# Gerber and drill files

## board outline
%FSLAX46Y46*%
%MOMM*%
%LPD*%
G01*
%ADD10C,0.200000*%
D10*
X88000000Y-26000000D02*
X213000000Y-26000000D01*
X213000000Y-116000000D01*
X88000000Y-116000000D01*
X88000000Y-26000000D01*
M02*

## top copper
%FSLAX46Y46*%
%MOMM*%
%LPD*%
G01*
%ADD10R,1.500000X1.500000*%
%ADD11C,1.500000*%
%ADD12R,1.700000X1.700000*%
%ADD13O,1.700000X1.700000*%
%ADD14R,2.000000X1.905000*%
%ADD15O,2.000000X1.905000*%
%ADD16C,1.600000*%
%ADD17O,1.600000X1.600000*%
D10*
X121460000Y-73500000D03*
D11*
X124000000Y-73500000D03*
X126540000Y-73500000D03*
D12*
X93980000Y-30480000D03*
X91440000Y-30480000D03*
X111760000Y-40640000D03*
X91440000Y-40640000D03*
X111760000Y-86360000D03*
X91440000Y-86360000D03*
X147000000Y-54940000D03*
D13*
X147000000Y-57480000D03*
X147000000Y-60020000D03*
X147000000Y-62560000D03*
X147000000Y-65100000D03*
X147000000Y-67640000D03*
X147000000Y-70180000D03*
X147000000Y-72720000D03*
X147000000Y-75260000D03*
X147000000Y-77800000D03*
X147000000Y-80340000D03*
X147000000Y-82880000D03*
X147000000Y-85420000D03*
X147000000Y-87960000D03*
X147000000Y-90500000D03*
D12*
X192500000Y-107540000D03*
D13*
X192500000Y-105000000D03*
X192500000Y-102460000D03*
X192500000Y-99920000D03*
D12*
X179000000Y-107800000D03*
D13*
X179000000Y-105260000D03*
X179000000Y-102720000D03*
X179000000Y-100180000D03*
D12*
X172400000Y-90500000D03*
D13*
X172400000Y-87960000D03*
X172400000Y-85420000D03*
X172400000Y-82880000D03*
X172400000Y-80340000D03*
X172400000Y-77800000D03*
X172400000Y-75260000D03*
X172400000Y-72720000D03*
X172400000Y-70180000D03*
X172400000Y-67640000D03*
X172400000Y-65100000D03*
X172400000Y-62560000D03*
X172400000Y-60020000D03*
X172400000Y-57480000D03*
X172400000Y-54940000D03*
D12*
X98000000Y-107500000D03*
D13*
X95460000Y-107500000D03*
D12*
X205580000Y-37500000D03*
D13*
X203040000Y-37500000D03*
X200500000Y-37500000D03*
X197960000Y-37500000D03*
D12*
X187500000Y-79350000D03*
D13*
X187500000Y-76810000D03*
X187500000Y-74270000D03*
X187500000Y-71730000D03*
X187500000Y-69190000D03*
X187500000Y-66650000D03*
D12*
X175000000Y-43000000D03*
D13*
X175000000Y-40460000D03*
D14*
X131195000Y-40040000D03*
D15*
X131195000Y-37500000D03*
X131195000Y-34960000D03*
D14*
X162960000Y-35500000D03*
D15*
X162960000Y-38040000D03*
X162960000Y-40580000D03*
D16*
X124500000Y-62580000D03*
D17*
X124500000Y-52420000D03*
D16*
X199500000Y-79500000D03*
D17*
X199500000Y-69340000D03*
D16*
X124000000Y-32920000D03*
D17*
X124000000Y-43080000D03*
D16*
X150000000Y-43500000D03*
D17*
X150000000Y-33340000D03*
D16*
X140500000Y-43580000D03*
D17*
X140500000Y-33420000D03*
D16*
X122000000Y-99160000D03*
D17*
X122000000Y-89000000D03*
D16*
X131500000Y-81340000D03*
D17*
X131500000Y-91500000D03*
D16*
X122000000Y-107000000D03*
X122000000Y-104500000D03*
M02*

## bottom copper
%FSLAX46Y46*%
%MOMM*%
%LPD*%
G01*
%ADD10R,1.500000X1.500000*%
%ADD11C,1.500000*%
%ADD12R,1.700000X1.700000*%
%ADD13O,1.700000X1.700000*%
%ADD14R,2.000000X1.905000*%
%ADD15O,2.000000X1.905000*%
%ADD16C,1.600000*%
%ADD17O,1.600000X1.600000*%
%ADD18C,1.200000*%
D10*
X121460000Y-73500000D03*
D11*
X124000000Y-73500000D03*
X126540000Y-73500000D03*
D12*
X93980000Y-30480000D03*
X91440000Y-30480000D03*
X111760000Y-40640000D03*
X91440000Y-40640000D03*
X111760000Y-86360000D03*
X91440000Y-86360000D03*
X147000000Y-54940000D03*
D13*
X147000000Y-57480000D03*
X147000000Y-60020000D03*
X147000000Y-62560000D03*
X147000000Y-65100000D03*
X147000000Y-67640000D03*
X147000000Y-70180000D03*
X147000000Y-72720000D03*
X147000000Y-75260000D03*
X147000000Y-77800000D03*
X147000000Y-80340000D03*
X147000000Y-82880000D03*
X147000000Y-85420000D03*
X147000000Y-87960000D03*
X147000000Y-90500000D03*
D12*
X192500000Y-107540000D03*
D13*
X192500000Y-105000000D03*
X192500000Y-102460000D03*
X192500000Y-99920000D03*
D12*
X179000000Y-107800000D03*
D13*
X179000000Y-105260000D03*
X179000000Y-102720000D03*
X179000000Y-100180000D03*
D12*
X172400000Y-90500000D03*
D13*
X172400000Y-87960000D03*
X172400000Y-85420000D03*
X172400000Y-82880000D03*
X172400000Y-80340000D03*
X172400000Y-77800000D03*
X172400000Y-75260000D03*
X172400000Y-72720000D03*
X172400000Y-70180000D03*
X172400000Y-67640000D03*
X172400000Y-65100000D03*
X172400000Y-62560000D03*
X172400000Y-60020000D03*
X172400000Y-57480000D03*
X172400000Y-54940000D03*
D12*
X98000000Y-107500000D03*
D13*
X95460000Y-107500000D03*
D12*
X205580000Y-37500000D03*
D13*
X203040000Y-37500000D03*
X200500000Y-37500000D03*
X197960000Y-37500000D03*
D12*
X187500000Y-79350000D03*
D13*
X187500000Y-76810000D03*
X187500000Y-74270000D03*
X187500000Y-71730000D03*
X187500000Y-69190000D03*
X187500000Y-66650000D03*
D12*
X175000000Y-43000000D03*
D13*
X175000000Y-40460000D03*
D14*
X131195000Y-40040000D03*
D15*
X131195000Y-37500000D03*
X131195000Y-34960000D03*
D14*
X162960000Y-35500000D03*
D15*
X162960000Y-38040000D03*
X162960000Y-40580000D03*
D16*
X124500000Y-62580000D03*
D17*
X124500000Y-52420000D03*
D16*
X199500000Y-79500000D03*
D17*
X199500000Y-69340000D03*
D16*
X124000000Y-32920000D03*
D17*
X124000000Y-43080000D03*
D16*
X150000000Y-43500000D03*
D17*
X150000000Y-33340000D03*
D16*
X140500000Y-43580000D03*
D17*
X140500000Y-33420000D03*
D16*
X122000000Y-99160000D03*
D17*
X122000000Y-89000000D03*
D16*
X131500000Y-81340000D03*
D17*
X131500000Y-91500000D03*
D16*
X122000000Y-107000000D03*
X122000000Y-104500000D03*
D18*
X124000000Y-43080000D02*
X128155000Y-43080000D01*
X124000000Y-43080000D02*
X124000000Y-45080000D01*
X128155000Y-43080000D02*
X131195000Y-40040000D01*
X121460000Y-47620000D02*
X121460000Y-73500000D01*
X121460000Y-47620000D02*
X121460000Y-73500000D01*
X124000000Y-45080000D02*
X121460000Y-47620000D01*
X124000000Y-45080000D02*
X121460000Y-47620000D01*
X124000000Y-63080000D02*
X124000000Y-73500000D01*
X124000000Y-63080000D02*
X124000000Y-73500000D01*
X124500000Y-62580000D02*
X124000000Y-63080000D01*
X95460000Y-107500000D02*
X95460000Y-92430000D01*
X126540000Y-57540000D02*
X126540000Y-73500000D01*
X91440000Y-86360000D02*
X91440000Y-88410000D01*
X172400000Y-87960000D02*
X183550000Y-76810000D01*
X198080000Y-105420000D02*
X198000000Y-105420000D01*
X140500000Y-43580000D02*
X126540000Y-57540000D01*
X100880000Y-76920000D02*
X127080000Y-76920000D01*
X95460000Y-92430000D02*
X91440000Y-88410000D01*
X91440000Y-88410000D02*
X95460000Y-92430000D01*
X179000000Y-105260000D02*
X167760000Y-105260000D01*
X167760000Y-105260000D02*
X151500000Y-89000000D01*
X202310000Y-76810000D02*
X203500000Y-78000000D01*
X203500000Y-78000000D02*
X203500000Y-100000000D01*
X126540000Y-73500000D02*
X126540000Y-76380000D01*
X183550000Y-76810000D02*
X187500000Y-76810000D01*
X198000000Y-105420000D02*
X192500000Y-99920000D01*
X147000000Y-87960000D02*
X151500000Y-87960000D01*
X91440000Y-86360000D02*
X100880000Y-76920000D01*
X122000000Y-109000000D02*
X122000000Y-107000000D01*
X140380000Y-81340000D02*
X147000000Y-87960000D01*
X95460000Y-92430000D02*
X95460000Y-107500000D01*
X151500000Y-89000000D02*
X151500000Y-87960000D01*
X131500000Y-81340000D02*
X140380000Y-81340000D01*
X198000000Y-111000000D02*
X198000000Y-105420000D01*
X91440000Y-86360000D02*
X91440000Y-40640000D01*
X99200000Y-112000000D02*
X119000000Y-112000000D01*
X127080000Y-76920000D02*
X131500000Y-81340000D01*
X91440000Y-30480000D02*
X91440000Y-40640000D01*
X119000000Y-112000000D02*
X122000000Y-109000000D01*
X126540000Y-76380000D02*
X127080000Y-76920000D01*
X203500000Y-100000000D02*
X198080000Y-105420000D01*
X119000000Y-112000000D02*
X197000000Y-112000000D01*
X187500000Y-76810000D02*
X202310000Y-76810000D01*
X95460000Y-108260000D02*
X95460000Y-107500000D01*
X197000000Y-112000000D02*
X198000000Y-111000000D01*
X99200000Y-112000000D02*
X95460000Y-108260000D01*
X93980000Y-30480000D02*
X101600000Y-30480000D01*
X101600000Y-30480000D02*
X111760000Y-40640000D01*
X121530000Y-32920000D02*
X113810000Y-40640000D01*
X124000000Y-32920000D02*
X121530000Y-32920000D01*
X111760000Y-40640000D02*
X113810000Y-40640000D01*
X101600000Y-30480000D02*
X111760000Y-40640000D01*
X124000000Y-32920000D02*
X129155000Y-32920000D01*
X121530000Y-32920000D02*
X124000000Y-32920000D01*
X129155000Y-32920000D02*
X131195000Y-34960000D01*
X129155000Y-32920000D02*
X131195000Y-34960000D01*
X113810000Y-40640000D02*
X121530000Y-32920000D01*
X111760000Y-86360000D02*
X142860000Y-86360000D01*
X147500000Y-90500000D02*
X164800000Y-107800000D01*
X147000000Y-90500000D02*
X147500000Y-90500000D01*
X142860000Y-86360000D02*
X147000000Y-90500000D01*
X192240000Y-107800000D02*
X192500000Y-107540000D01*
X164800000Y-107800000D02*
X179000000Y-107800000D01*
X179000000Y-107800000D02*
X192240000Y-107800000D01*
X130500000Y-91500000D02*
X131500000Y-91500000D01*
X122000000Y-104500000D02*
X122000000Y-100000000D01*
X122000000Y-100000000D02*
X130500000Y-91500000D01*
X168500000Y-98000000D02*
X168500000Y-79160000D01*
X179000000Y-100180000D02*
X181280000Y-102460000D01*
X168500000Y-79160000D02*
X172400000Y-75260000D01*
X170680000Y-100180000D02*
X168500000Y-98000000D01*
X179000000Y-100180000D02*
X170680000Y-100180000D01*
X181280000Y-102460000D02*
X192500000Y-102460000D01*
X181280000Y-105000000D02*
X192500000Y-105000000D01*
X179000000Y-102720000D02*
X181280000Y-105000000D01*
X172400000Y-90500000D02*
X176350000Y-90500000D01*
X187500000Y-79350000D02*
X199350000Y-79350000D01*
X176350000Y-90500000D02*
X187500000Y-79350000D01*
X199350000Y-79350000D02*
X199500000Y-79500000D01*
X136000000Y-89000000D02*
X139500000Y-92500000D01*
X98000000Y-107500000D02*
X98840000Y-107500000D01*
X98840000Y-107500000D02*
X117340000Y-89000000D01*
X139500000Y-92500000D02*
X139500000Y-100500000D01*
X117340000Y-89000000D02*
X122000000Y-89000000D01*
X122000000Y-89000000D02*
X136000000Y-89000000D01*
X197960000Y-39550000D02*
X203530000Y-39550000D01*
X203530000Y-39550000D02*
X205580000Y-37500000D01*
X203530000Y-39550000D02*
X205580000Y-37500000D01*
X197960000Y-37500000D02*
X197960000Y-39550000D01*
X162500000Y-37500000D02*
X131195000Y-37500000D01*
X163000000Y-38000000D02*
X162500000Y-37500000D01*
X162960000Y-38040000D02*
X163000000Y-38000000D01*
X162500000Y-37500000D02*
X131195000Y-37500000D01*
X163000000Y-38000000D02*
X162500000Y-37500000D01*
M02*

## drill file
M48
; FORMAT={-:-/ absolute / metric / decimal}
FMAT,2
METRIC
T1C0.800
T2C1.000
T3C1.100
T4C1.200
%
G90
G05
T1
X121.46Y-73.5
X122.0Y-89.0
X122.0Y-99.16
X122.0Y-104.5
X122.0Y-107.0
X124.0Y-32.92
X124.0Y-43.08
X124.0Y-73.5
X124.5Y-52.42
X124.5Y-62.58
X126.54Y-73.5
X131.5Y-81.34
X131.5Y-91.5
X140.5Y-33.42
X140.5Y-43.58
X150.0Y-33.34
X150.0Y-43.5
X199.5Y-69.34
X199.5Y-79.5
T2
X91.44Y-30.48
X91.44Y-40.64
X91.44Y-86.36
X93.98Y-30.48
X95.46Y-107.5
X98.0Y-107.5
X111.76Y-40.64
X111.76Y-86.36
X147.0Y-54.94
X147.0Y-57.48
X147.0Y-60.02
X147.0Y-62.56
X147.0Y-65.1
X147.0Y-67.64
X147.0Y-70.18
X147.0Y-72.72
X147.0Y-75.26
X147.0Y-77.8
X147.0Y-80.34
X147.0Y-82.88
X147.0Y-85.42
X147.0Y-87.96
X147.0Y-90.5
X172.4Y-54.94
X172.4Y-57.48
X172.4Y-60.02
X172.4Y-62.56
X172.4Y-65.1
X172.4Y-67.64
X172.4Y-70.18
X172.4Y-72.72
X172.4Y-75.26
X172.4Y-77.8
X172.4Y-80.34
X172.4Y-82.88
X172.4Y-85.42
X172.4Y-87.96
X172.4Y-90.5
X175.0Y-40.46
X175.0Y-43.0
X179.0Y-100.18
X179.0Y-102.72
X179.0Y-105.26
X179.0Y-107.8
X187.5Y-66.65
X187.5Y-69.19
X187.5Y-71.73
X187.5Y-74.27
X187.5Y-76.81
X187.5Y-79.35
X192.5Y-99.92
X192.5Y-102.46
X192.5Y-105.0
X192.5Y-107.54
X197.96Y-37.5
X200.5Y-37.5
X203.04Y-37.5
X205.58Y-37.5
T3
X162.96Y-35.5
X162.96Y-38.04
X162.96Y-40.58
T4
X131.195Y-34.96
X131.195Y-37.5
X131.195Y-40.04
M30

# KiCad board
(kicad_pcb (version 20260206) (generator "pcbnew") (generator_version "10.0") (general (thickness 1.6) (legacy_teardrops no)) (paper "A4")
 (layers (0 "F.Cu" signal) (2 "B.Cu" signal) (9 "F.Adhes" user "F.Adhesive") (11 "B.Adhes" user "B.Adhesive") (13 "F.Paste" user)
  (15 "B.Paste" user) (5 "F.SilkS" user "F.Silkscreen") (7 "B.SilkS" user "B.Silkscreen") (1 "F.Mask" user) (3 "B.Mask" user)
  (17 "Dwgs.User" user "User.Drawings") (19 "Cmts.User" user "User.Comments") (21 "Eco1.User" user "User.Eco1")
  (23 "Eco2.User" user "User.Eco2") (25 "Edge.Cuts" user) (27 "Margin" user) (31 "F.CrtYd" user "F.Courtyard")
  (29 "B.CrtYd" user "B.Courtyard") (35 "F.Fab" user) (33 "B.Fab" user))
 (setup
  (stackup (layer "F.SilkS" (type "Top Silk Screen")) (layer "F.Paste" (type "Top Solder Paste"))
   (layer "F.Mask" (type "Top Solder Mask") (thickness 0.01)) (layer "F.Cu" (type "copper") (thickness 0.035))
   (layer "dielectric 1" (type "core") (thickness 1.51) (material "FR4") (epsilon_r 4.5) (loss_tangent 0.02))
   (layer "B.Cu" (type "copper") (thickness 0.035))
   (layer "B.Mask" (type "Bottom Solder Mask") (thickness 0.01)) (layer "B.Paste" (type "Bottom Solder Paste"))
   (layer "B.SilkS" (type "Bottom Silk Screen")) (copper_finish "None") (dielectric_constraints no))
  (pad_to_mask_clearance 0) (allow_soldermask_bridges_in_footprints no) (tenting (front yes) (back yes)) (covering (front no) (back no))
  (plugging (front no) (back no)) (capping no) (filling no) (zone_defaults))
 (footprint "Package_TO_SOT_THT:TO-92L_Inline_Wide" (layer "F.Cu") (at 121.46 73.5)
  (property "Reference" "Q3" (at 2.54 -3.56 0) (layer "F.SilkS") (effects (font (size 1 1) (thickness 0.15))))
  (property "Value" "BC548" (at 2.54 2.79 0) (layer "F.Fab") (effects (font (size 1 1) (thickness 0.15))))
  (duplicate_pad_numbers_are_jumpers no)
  (pad "1" thru_hole rect (at 0 0) (size 1.5 1.5) (drill 0.8) (layers "*.Cu" "*.Mask") (remove_unused_layers no) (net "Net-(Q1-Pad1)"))
  (pad "2" thru_hole circle (at 2.54 0) (size 1.5 1.5) (drill 0.8) (layers "*.Cu" "*.Mask") (remove_unused_layers no) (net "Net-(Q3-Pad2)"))
  (pad "3" thru_hole circle (at 5.08 0) (size 1.5 1.5) (drill 0.8) (layers "*.Cu" "*.Mask") (remove_unused_layers no) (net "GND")))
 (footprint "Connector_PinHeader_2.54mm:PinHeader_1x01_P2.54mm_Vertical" (layer "F.Cu") (at 93.98 30.48)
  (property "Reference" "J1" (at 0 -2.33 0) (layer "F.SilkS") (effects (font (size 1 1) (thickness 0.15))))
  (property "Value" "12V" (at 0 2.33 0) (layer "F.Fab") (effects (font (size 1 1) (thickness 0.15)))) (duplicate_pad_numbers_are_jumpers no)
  (pad "1" thru_hole rect (at 0 0) (size 1.7 1.7) (drill 1) (layers "*.Cu" "*.Mask") (remove_unused_layers no) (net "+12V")))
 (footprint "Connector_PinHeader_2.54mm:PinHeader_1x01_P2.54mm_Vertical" (layer "F.Cu") (at 91.44 30.48)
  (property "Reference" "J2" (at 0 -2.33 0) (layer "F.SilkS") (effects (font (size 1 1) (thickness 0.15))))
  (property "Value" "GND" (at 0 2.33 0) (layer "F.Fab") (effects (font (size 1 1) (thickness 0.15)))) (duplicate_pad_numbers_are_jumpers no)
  (pad "1" thru_hole rect (at 0 0) (size 1.7 1.7) (drill 1) (layers "*.Cu" "*.Mask") (remove_unused_layers no) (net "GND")))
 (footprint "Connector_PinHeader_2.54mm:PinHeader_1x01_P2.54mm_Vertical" (layer "F.Cu") (at 111.76 40.64)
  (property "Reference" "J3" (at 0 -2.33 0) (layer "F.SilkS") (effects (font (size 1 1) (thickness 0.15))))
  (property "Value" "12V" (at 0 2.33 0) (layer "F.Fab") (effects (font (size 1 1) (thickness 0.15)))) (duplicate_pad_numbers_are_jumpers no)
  (pad "1" thru_hole rect (at 0 0) (size 1.7 1.7) (drill 1) (layers "*.Cu" "*.Mask") (remove_unused_layers no) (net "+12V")))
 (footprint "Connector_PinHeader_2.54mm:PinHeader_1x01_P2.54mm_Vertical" (layer "F.Cu") (at 91.44 40.64)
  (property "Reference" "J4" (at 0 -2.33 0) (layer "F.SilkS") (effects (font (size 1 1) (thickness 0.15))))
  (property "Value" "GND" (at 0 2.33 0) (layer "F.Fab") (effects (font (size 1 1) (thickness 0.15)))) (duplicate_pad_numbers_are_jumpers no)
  (pad "1" thru_hole rect (at 0 0) (size 1.7 1.7) (drill 1) (layers "*.Cu" "*.Mask") (remove_unused_layers no) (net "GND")))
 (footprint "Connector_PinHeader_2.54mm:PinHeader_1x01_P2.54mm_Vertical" (layer "F.Cu") (at 111.76 86.36)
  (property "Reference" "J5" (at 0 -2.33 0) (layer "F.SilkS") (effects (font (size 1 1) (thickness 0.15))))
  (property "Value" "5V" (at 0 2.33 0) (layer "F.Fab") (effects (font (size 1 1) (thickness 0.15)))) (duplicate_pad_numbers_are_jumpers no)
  (pad "1" thru_hole rect (at 0 0) (size 1.7 1.7) (drill 1) (layers "*.Cu" "*.Mask") (remove_unused_layers no) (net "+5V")))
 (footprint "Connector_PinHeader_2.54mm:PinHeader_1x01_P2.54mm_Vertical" (layer "F.Cu") (at 91.44 86.36)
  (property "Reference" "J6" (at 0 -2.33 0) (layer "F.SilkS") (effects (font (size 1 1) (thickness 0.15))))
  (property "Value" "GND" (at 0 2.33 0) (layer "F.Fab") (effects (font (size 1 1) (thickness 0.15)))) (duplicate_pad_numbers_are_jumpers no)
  (pad "1" thru_hole rect (at 0 0) (size 1.7 1.7) (drill 1) (layers "*.Cu" "*.Mask") (remove_unused_layers no) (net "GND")))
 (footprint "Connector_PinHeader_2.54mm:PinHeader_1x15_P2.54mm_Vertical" (layer "F.Cu") (at 147 54.94)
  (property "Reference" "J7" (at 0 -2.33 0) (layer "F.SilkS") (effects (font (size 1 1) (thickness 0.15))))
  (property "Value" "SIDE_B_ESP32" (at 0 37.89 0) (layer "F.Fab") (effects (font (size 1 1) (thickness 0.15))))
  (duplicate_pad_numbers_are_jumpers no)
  (pad "1" thru_hole rect (at 0 0) (size 1.7 1.7) (drill 1) (layers "*.Cu" "*.Mask") (remove_unused_layers no) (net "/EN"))
  (pad "2" thru_hole oval (at 0 2.54) (size 1.7 1.7) (drill 1) (layers "*.Cu" "*.Mask") (remove_unused_layers no) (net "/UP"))
  (pad "3" thru_hole oval (at 0 5.08) (size 1.7 1.7) (drill 1) (layers "*.Cu" "*.Mask") (remove_unused_layers no) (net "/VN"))
  (pad "4" thru_hole oval (at 0 7.62) (size 1.7 1.7) (drill 1) (layers "*.Cu" "*.Mask") (remove_unused_layers no) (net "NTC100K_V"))
  (pad "5" thru_hole oval (at 0 10.16) (size 1.7 1.7) (drill 1) (layers "*.Cu" "*.Mask") (remove_unused_layers no) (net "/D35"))
  (pad "6" thru_hole oval (at 0 12.7) (size 1.7 1.7) (drill 1) (layers "*.Cu" "*.Mask") (remove_unused_layers no) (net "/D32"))
  (pad "7" thru_hole oval (at 0 15.24) (size 1.7 1.7) (drill 1) (layers "*.Cu" "*.Mask") (remove_unused_layers no) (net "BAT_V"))
  (pad "8" thru_hole oval (at 0 17.78) (size 1.7 1.7) (drill 1) (layers "*.Cu" "*.Mask") (remove_unused_layers no) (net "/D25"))
  (pad "9" thru_hole oval (at 0 20.32) (size 1.7 1.7) (drill 1) (layers "*.Cu" "*.Mask") (remove_unused_layers no) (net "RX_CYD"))
  (pad "10" thru_hole oval (at 0 22.86) (size 1.7 1.7) (drill 1) (layers "*.Cu" "*.Mask") (remove_unused_layers no) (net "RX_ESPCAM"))
  (pad "11" thru_hole oval (at 0 25.4) (size 1.7 1.7) (drill 1) (layers "*.Cu" "*.Mask") (remove_unused_layers no) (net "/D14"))
  (pad "12" thru_hole oval (at 0 27.94) (size 1.7 1.7) (drill 1) (layers "*.Cu" "*.Mask") (remove_unused_layers no) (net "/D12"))
  (pad "13" thru_hole oval (at 0 30.48) (size 1.7 1.7) (drill 1) (layers "*.Cu" "*.Mask") (remove_unused_layers no) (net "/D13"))
  (pad "14" thru_hole oval (at 0 33.02) (size 1.7 1.7) (drill 1) (layers "*.Cu" "*.Mask") (remove_unused_layers no) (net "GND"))
  (pad "15" thru_hole oval (at 0 35.56) (size 1.7 1.7) (drill 1) (layers "*.Cu" "*.Mask") (remove_unused_layers no) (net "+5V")))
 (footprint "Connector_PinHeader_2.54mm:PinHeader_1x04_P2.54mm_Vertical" (layer "F.Cu") (at 192.5 107.54 180)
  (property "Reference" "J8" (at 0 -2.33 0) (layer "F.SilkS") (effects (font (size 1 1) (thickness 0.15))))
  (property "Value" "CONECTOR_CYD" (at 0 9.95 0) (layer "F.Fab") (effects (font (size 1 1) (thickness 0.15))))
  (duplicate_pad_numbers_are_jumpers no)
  (pad "1" thru_hole rect (at 0 0 180) (size 1.7 1.7) (drill 1) (layers "*.Cu" "*.Mask") (remove_unused_layers no) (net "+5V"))
  (pad "2" thru_hole oval (at 0 2.54 180) (size 1.7 1.7) (drill 1) (layers "*.Cu" "*.Mask") (remove_unused_layers no) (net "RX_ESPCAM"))
  (pad "3" thru_hole oval (at 0 5.08 180) (size 1.7 1.7) (drill 1) (layers "*.Cu" "*.Mask") (remove_unused_layers no) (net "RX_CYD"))
  (pad "4" thru_hole oval (at 0 7.62 180) (size 1.7 1.7) (drill 1) (layers "*.Cu" "*.Mask") (remove_unused_layers no) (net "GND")))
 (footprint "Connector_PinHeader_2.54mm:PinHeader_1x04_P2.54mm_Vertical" (layer "F.Cu") (at 179 107.8 180)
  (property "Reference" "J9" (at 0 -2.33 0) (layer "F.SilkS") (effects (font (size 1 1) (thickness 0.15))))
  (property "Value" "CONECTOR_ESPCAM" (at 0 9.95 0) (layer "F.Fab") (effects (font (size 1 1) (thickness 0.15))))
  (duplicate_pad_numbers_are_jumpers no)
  (pad "1" thru_hole rect (at 0 0 180) (size 1.7 1.7) (drill 1) (layers "*.Cu" "*.Mask") (remove_unused_layers no) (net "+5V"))
  (pad "2" thru_hole oval (at 0 2.54 180) (size 1.7 1.7) (drill 1) (layers "*.Cu" "*.Mask") (remove_unused_layers no) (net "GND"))
  (pad "3" thru_hole oval (at 0 5.08 180) (size 1.7 1.7) (drill 1) (layers "*.Cu" "*.Mask") (remove_unused_layers no) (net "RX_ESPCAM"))
  (pad "4" thru_hole oval (at 0 7.62 180) (size 1.7 1.7) (drill 1) (layers "*.Cu" "*.Mask") (remove_unused_layers no) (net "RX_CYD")))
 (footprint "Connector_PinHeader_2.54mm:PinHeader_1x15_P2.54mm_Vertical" (layer "F.Cu") (at 172.4 90.5 180)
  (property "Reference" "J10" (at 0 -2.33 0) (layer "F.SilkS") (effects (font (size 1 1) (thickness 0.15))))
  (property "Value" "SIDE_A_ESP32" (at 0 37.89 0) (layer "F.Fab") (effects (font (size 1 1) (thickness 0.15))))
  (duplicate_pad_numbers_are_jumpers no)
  (pad "1" thru_hole rect (at 0 0 180) (size 1.7 1.7) (drill 1) (layers "*.Cu" "*.Mask") (remove_unused_layers no) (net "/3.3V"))
  (pad "2" thru_hole oval (at 0 2.54 180) (size 1.7 1.7) (drill 1) (layers "*.Cu" "*.Mask") (remove_unused_layers no) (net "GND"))
  (pad "3" thru_hole oval (at 0 5.08 180) (size 1.7 1.7) (drill 1) (layers "*.Cu" "*.Mask") (remove_unused_layers no) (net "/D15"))
  (pad "4" thru_hole oval (at 0 7.62 180) (size 1.7 1.7) (drill 1) (layers "*.Cu" "*.Mask") (remove_unused_layers no) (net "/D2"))
  (pad "5" thru_hole oval (at 0 10.16 180) (size 1.7 1.7) (drill 1) (layers "*.Cu" "*.Mask") (remove_unused_layers no) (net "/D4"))
  (pad "6" thru_hole oval (at 0 12.7 180) (size 1.7 1.7) (drill 1) (layers "*.Cu" "*.Mask") (remove_unused_layers no) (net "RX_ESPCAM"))
  (pad "7" thru_hole oval (at 0 15.24 180) (size 1.7 1.7) (drill 1) (layers "*.Cu" "*.Mask") (remove_unused_layers no) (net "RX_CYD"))
  (pad "8" thru_hole oval (at 0 17.78 180) (size 1.7 1.7) (drill 1) (layers "*.Cu" "*.Mask") (remove_unused_layers no) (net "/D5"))
  (pad "9" thru_hole oval (at 0 20.32 180) (size 1.7 1.7) (drill 1) (layers "*.Cu" "*.Mask") (remove_unused_layers no) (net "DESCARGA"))
  (pad "10" thru_hole oval (at 0 22.86 180) (size 1.7 1.7) (drill 1) (layers "*.Cu" "*.Mask") (remove_unused_layers no) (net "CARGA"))
  (pad "11" thru_hole oval (at 0 25.4 180) (size 1.7 1.7) (drill 1) (layers "*.Cu" "*.Mask") (remove_unused_layers no) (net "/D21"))
  (pad "12" thru_hole oval (at 0 27.94 180) (size 1.7 1.7) (drill 1) (layers "*.Cu" "*.Mask") (remove_unused_layers no) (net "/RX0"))
  (pad "13" thru_hole oval (at 0 30.48 180) (size 1.7 1.7) (drill 1) (layers "*.Cu" "*.Mask") (remove_unused_layers no) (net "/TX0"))
  (pad "14" thru_hole oval (at 0 33.02 180) (size 1.7 1.7) (drill 1) (layers "*.Cu" "*.Mask") (remove_unused_layers no) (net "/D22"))
  (pad "15" thru_hole oval (at 0 35.56 180) (size 1.7 1.7) (drill 1) (layers "*.Cu" "*.Mask") (remove_unused_layers no) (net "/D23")))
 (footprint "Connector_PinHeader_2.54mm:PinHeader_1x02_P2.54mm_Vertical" (layer "F.Cu") (at 98 107.5 -90)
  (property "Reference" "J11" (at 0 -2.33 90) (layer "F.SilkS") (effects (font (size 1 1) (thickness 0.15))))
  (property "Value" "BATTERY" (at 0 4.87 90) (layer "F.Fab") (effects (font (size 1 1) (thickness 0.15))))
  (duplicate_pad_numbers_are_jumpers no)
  (pad "1" thru_hole rect (at 0 0 270) (size 1.7 1.7) (drill 1) (layers "*.Cu" "*.Mask") (remove_unused_layers no) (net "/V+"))
  (pad "2" thru_hole oval (at 0 2.54 270) (size 1.7 1.7) (drill 1) (layers "*.Cu" "*.Mask") (remove_unused_layers no) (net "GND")))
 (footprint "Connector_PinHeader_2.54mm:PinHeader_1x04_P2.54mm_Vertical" (layer "F.Cu") (at 205.58 37.5 -90)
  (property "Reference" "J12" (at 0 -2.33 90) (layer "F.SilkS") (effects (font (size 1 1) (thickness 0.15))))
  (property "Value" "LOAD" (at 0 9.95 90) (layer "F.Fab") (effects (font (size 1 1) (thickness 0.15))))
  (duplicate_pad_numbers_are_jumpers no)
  (pad "1" thru_hole rect (at 0 0 270) (size 1.7 1.7) (drill 1) (layers "*.Cu" "*.Mask") (remove_unused_layers no) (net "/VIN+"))
  (pad "2" thru_hole oval (at 0 2.54 270) (size 1.7 1.7) (drill 1) (layers "*.Cu" "*.Mask") (remove_unused_layers no) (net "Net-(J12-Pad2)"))
  (pad "3" thru_hole oval (at 0 5.08 270) (size 1.7 1.7) (drill 1) (layers "*.Cu" "*.Mask") (remove_unused_layers no) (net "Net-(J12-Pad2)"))
  (pad "4" thru_hole oval (at 0 7.62 270) (size 1.7 1.7) (drill 1) (layers "*.Cu" "*.Mask") (remove_unused_layers no) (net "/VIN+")))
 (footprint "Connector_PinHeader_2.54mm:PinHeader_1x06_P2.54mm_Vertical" (layer "F.Cu") (at 187.5 79.35 180)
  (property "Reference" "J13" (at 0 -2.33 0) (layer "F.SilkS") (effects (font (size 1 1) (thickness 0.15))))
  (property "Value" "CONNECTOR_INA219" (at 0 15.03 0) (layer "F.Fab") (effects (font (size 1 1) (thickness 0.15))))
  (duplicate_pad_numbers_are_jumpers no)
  (pad "1" thru_hole rect (at 0 0 180) (size 1.7 1.7) (drill 1) (layers "*.Cu" "*.Mask") (remove_unused_layers no) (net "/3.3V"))
  (pad "2" thru_hole oval (at 0 2.54 180) (size 1.7 1.7) (drill 1) (layers "*.Cu" "*.Mask") (remove_unused_layers no) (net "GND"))
  (pad "3" thru_hole oval (at 0 5.08 180) (size 1.7 1.7) (drill 1) (layers "*.Cu" "*.Mask") (remove_unused_layers no) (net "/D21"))
  (pad "4" thru_hole oval (at 0 7.62 180) (size 1.7 1.7) (drill 1) (layers "*.Cu" "*.Mask") (remove_unused_layers no) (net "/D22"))
  (pad "5" thru_hole oval (at 0 10.16 180) (size 1.7 1.7) (drill 1) (layers "*.Cu" "*.Mask") (remove_unused_layers no) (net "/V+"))
  (pad "6" thru_hole oval (at 0 12.7 180) (size 1.7 1.7) (drill 1) (layers "*.Cu" "*.Mask") (remove_unused_layers no) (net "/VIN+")))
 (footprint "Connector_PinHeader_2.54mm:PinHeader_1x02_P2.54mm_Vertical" (layer "F.Cu") (at 175 43 180)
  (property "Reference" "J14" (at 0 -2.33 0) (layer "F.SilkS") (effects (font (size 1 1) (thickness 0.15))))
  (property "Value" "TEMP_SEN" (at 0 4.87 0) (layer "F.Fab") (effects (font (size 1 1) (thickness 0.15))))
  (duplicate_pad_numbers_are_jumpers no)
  (pad "1" thru_hole rect (at 0 0 180) (size 1.7 1.7) (drill 1) (layers "*.Cu" "*.Mask") (remove_unused_layers no) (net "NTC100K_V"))
  (pad "2" thru_hole oval (at 0 2.54 180) (size 1.7 1.7) (drill 1) (layers "*.Cu" "*.Mask") (remove_unused_layers no) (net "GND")))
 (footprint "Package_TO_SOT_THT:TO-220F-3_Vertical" (layer "F.Cu") (at 131.195 40.04 90)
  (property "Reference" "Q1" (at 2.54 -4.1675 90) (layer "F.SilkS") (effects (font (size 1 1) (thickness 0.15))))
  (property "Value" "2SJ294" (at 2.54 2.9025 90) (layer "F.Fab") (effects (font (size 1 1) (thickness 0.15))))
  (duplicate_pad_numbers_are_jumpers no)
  (pad "1" thru_hole rect (at 0 0 90) (size 1.905 2) (drill 1.2) (layers "*.Cu" "*.Mask") (remove_unused_layers no) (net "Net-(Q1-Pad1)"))
  (pad "2" thru_hole oval (at 2.54 0 90) (size 1.905 2) (drill 1.2) (layers "*.Cu" "*.Mask") (remove_unused_layers no)
   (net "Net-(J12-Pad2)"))
  (pad "3" thru_hole oval (at 5.08 0 90) (size 1.905 2) (drill 1.2) (layers "*.Cu" "*.Mask") (remove_unused_layers no) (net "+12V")))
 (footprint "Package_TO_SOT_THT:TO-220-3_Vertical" (layer "F.Cu") (at 162.96 35.5 -90)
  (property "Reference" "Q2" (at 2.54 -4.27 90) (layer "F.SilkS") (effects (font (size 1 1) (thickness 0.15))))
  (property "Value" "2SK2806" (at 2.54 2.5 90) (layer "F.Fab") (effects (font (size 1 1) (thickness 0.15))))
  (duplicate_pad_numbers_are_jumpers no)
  (pad "1" thru_hole rect (at 0 0 270) (size 1.905 2) (drill 1.1) (layers "*.Cu" "*.Mask") (remove_unused_layers no) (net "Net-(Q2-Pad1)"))
  (pad "2" thru_hole oval (at 2.54 0 270) (size 1.905 2) (drill 1.1) (layers "*.Cu" "*.Mask") (remove_unused_layers no)
   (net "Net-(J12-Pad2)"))
  (pad "3" thru_hole oval (at 5.08 0 270) (size 1.905 2) (drill 1.1) (layers "*.Cu" "*.Mask") (remove_unused_layers no) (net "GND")))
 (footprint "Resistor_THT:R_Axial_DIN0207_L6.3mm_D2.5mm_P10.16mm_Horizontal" (layer "F.Cu") (at 124.5 62.58 90)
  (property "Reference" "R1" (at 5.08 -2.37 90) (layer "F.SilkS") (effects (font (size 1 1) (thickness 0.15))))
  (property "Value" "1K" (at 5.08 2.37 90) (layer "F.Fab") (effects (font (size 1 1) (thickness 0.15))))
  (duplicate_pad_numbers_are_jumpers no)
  (pad "1" thru_hole circle (at 0 0 90) (size 1.6 1.6) (drill 0.8) (layers "*.Cu" "*.Mask") (remove_unused_layers no) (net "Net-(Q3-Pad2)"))
  (pad "2" thru_hole oval (at 10.16 0 90) (size 1.6 1.6) (drill 0.8) (layers "*.Cu" "*.Mask") (remove_unused_layers no) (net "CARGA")))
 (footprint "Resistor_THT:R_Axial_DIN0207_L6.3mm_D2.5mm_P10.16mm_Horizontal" (layer "F.Cu") (at 199.5 79.5 90)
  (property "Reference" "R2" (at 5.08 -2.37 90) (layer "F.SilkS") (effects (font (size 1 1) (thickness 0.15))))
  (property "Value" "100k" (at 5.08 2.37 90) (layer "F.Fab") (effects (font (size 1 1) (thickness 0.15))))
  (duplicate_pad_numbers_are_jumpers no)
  (pad "1" thru_hole circle (at 0 0 90) (size 1.6 1.6) (drill 0.8) (layers "*.Cu" "*.Mask") (remove_unused_layers no) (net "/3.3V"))
  (pad "2" thru_hole oval (at 10.16 0 90) (size 1.6 1.6) (drill 0.8) (layers "*.Cu" "*.Mask") (remove_unused_layers no) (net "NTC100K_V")))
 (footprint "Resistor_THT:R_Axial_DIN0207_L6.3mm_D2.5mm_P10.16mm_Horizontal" (layer "F.Cu") (at 124 32.92 -90)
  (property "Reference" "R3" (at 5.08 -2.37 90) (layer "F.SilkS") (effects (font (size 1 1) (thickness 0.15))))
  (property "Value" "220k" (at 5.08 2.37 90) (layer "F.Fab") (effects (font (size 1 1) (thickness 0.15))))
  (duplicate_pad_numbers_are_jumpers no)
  (pad "1" thru_hole circle (at 0 0 270) (size 1.6 1.6) (drill 0.8) (layers "*.Cu" "*.Mask") (remove_unused_layers no) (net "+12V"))
  (pad "2" thru_hole oval (at 10.16 0 270) (size 1.6 1.6) (drill 0.8) (layers "*.Cu" "*.Mask") (remove_unused_layers no)
   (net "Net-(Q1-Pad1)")))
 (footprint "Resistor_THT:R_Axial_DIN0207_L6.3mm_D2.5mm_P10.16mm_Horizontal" (layer "F.Cu") (at 150 43.5 90)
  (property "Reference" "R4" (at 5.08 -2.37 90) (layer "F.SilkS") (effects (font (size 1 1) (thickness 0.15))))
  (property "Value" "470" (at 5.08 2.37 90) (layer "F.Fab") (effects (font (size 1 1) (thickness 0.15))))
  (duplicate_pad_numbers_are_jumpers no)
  (pad "1" thru_hole circle (at 0 0 90) (size 1.6 1.6) (drill 0.8) (layers "*.Cu" "*.Mask") (remove_unused_layers no) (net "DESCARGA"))
  (pad "2" thru_hole oval (at 10.16 0 90) (size 1.6 1.6) (drill 0.8) (layers "*.Cu" "*.Mask") (remove_unused_layers no)
   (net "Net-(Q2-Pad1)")))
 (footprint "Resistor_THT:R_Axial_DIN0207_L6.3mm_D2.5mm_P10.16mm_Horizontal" (layer "F.Cu") (at 140.5 43.58 90)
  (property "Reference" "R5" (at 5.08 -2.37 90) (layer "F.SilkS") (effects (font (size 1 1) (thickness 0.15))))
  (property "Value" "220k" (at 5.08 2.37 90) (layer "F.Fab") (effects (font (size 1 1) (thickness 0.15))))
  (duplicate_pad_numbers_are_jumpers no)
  (pad "1" thru_hole circle (at 0 0 90) (size 1.6 1.6) (drill 0.8) (layers "*.Cu" "*.Mask") (remove_unused_layers no) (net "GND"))
  (pad "2" thru_hole oval (at 10.16 0 90) (size 1.6 1.6) (drill 0.8) (layers "*.Cu" "*.Mask") (remove_unused_layers no)
   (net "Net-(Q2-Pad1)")))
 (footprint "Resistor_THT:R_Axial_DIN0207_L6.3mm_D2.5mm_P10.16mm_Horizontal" (layer "F.Cu") (at 122 99.16 90)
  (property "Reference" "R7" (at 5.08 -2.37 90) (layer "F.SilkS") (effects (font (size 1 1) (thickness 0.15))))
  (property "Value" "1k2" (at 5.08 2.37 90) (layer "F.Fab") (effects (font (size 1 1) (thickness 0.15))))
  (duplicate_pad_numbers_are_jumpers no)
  (pad "1" thru_hole circle (at 0 0 90) (size 1.6 1.6) (drill 0.8) (layers "*.Cu" "*.Mask") (remove_unused_layers no) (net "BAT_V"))
  (pad "2" thru_hole oval (at 10.16 0 90) (size 1.6 1.6) (drill 0.8) (layers "*.Cu" "*.Mask") (remove_unused_layers no) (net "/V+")))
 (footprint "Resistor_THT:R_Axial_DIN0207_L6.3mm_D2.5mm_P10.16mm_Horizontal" (layer "F.Cu") (at 131.5 81.34 -90)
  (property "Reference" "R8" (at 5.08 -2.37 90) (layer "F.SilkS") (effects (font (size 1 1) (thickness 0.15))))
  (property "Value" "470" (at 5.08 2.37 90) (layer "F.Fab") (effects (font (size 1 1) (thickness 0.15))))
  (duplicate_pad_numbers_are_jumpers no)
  (pad "1" thru_hole circle (at 0 0 270) (size 1.6 1.6) (drill 0.8) (layers "*.Cu" "*.Mask") (remove_unused_layers no) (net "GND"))
  (pad "2" thru_hole oval (at 10.16 0 270) (size 1.6 1.6) (drill 0.8) (layers "*.Cu" "*.Mask") (remove_unused_layers no) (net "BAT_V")))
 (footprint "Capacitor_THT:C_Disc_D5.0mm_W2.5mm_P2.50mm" (layer "F.Cu") (at 122 107 90)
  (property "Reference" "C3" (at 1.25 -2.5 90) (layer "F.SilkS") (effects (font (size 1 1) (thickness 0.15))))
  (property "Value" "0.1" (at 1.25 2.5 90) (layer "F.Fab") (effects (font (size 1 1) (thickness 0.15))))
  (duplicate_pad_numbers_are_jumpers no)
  (pad "1" thru_hole circle (at 0 0 90) (size 1.6 1.6) (drill 0.8) (layers "*.Cu" "*.Mask") (remove_unused_layers no) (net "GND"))
  (pad "2" thru_hole circle (at 2.5 0 90) (size 1.6 1.6) (drill 0.8) (layers "*.Cu" "*.Mask") (remove_unused_layers no) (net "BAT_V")))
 (gr_rect (start 88 26) (end 213 116) (stroke (width 0.2) (type solid)) (fill no) (layer "Edge.Cuts"))
 (segment (start 124 43.08) (end 128.155 43.08) (width 1.2) (layer "B.Cu") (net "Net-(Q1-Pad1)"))
 (segment (start 124 43.08) (end 124 45.08) (width 1.2) (layer "B.Cu") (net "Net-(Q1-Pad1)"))
 (segment (start 128.155 43.08) (end 131.195 40.04) (width 1.2) (layer "B.Cu") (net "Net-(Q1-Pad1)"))
 (segment (start 121.46 47.62) (end 121.46 73.5) (width 1.2) (layer "B.Cu") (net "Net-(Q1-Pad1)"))
 (segment (start 121.46 47.62) (end 121.46 73.5) (width 1.2) (layer "B.Cu") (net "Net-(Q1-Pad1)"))
 (segment (start 124 45.08) (end 121.46 47.62) (width 1.2) (layer "B.Cu") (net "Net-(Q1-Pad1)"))
 (segment (start 124 45.08) (end 121.46 47.62) (width 1.2) (layer "B.Cu") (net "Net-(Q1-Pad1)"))
 (segment (start 124 63.08) (end 124 73.5) (width 1.2) (layer "B.Cu") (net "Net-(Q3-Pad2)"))
 (segment (start 124 63.08) (end 124 73.5) (width 1.2) (layer "B.Cu") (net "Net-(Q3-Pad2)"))
 (segment (start 124.5 62.58) (end 124 63.08) (width 1.2) (layer "B.Cu") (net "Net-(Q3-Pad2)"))
 (segment (start 95.46 107.5) (end 95.46 92.43) (width 1.2) (layer "B.Cu") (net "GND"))
 (segment (start 126.54 57.54) (end 126.54 73.5) (width 1.2) (layer "B.Cu") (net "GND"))
 (segment (start 91.44 86.36) (end 91.44 88.41) (width 1.2) (layer "B.Cu") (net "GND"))
 (segment (start 172.4 87.96) (end 183.55 76.81) (width 1.2) (layer "B.Cu") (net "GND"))
 (segment (start 198.08 105.42) (end 198 105.42) (width 1.2) (layer "B.Cu") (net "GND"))
 (segment (start 140.5 43.58) (end 126.54 57.54) (width 1.2) (layer "B.Cu") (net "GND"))
 (segment (start 100.88 76.92) (end 127.08 76.92) (width 1.2) (layer "B.Cu") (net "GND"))
 (segment (start 95.46 92.43) (end 91.44 88.41) (width 1.2) (layer "B.Cu") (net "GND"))
 (segment (start 91.44 88.41) (end 95.46 92.43) (width 1.2) (layer "B.Cu") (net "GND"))
 (segment (start 179 105.26) (end 167.76 105.26) (width 1.2) (layer "B.Cu") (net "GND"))
 (segment (start 167.76 105.26) (end 151.5 89) (width 1.2) (layer "B.Cu") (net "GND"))
 (segment (start 202.31 76.81) (end 203.5 78) (width 1.2) (layer "B.Cu") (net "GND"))
 (segment (start 203.5 78) (end 203.5 100) (width 1.2) (layer "B.Cu") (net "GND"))
 (segment (start 126.54 73.5) (end 126.54 76.38) (width 1.2) (layer "B.Cu") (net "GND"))
 (segment (start 183.55 76.81) (end 187.5 76.81) (width 1.2) (layer "B.Cu") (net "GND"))
 (segment (start 198 105.42) (end 192.5 99.92) (width 1.2) (layer "B.Cu") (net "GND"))
 (segment (start 147 87.96) (end 151.5 87.96) (width 1.2) (layer "B.Cu") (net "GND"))
 (segment (start 91.44 86.36) (end 100.88 76.92) (width 1.2) (layer "B.Cu") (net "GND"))
 (segment (start 122 109) (end 122 107) (width 1.2) (layer "B.Cu") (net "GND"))
 (segment (start 140.38 81.34) (end 147 87.96) (width 1.2) (layer "B.Cu") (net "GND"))
 (segment (start 95.46 92.43) (end 95.46 107.5) (width 1.2) (layer "B.Cu") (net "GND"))
 (segment (start 151.5 89) (end 151.5 87.96) (width 1.2) (layer "B.Cu") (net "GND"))
 (segment (start 131.5 81.34) (end 140.38 81.34) (width 1.2) (layer "B.Cu") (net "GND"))
 (segment (start 198 111) (end 198 105.42) (width 1.2) (layer "B.Cu") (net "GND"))
 (segment (start 91.44 86.36) (end 91.44 40.64) (width 1.2) (layer "B.Cu") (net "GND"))
 (segment (start 99.2 112) (end 119 112) (width 1.2) (layer "B.Cu") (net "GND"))
 (segment (start 127.08 76.92) (end 131.5 81.34) (width 1.2) (layer "B.Cu") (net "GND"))
 (segment (start 91.44 30.48) (end 91.44 40.64) (width 1.2) (layer "B.Cu") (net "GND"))
 (segment (start 119 112) (end 122 109) (width 1.2) (layer "B.Cu") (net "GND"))
 (segment (start 126.54 76.38) (end 127.08 76.92) (width 1.2) (layer "B.Cu") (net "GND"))
 (segment (start 203.5 100) (end 198.08 105.42) (width 1.2) (layer "B.Cu") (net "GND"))
 (segment (start 119 112) (end 197 112) (width 1.2) (layer "B.Cu") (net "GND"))
 (segment (start 187.5 76.81) (end 202.31 76.81) (width 1.2) (layer "B.Cu") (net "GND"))
 (segment (start 95.46 108.26) (end 95.46 107.5) (width 1.2) (layer "B.Cu") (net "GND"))
 (segment (start 197 112) (end 198 111) (width 1.2) (layer "B.Cu") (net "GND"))
 (segment (start 99.2 112) (end 95.46 108.26) (width 1.2) (layer "B.Cu") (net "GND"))
 (segment (start 93.98 30.48) (end 101.6 30.48) (width 1.2) (layer "B.Cu") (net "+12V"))
 (segment (start 101.6 30.48) (end 111.76 40.64) (width 1.2) (layer "B.Cu") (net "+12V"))
 (segment (start 121.53 32.92) (end 113.81 40.64) (width 1.2) (layer "B.Cu") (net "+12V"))
 (segment (start 124 32.92) (end 121.53 32.92) (width 1.2) (layer "B.Cu") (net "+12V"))
 (segment (start 111.76 40.64) (end 113.81 40.64) (width 1.2) (layer "B.Cu") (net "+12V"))
 (segment (start 101.6 30.48) (end 111.76 40.64) (width 1.2) (layer "B.Cu") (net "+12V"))
 (segment (start 124 32.92) (end 129.155 32.92) (width 1.2) (layer "B.Cu") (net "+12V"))
 (segment (start 121.53 32.92) (end 124 32.92) (width 1.2) (layer "B.Cu") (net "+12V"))
 (segment (start 129.155 32.92) (end 131.195 34.96) (width 1.2) (layer "B.Cu") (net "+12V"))
 (segment (start 129.155 32.92) (end 131.195 34.96) (width 1.2) (layer "B.Cu") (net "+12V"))
 (segment (start 113.81 40.64) (end 121.53 32.92) (width 1.2) (layer "B.Cu") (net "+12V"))
 (segment (start 111.76 86.36) (end 142.86 86.36) (width 1.2) (layer "B.Cu") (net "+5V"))
 (segment (start 147.5 90.5) (end 164.8 107.8) (width 1.2) (layer "B.Cu") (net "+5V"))
 (segment (start 147 90.5) (end 147.5 90.5) (width 1.2) (layer "B.Cu") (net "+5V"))
 (segment (start 142.86 86.36) (end 147 90.5) (width 1.2) (layer "B.Cu") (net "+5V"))
 (segment (start 192.24 107.8) (end 192.5 107.54) (width 1.2) (layer "B.Cu") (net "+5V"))
 (segment (start 164.8 107.8) (end 179 107.8) (width 1.2) (layer "B.Cu") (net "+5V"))
 (segment (start 179 107.8) (end 192.24 107.8) (width 1.2) (layer "B.Cu") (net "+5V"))
 (segment (start 130.5 91.5) (end 131.5 91.5) (width 1.2) (layer "B.Cu") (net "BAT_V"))
 (segment (start 122 104.5) (end 122 100) (width 1.2) (layer "B.Cu") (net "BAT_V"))
 (segment (start 122 100) (end 130.5 91.5) (width 1.2) (layer "B.Cu") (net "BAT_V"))
 (segment (start 168.5 98) (end 168.5 79.16) (width 1.2) (layer "B.Cu") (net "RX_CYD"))
 (segment (start 179 100.18) (end 181.28 102.46) (width 1.2) (layer "B.Cu") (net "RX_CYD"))
 (segment (start 168.5 79.16) (end 172.4 75.26) (width 1.2) (layer "B.Cu") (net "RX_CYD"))
 (segment (start 170.68 100.18) (end 168.5 98) (width 1.2) (layer "B.Cu") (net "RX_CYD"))
 (segment (start 179 100.18) (end 170.68 100.18) (width 1.2) (layer "B.Cu") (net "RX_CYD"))
 (segment (start 181.28 102.46) (end 192.5 102.46) (width 1.2) (layer "B.Cu") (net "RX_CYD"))
 (segment (start 181.28 105) (end 192.5 105) (width 1.2) (layer "B.Cu") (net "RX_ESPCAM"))
 (segment (start 179 102.72) (end 181.28 105) (width 1.2) (layer "B.Cu") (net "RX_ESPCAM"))
 (segment (start 172.4 90.5) (end 176.35 90.5) (width 1.2) (layer "B.Cu") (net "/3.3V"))
 (segment (start 187.5 79.35) (end 199.35 79.35) (width 1.2) (layer "B.Cu") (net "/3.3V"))
 (segment (start 176.35 90.5) (end 187.5 79.35) (width 1.2) (layer "B.Cu") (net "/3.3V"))
 (segment (start 199.35 79.35) (end 199.5 79.5) (width 1.2) (layer "B.Cu") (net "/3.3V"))
 (segment (start 136 89) (end 139.5 92.5) (width 1.2) (layer "B.Cu") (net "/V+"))
 (segment (start 98 107.5) (end 98.84 107.5) (width 1.2) (layer "B.Cu") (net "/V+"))
 (segment (start 98.84 107.5) (end 117.34 89) (width 1.2) (layer "B.Cu") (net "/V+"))
 (segment (start 139.5 92.5) (end 139.5 100.5) (width 1.2) (layer "B.Cu") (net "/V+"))
 (segment (start 117.34 89) (end 122 89) (width 1.2) (layer "B.Cu") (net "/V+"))
 (segment (start 122 89) (end 136 89) (width 1.2) (layer "B.Cu") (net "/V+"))
 (segment (start 197.96 39.55) (end 203.53 39.55) (width 1.2) (layer "B.Cu") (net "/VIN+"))
 (segment (start 203.53 39.55) (end 205.58 37.5) (width 1.2) (layer "B.Cu") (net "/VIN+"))
 (segment (start 203.53 39.55) (end 205.58 37.5) (width 1.2) (layer "B.Cu") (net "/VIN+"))
 (segment (start 197.96 37.5) (end 197.96 39.55) (width 1.2) (layer "B.Cu") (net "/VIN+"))
 (segment (start 162.5 37.5) (end 131.195 37.5) (width 1.2) (layer "B.Cu") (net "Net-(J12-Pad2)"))
 (segment (start 163 38) (end 162.5 37.5) (width 1.2) (layer "B.Cu") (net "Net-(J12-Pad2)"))
 (segment (start 162.96 38.04) (end 163 38) (width 1.2) (layer "B.Cu") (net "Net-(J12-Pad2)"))
 (segment (start 162.5 37.5) (end 131.195 37.5) (width 1.2) (layer "B.Cu") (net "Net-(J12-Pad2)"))
 (segment (start 163 38) (end 162.5 37.5) (width 1.2) (layer "B.Cu") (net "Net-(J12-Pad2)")))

